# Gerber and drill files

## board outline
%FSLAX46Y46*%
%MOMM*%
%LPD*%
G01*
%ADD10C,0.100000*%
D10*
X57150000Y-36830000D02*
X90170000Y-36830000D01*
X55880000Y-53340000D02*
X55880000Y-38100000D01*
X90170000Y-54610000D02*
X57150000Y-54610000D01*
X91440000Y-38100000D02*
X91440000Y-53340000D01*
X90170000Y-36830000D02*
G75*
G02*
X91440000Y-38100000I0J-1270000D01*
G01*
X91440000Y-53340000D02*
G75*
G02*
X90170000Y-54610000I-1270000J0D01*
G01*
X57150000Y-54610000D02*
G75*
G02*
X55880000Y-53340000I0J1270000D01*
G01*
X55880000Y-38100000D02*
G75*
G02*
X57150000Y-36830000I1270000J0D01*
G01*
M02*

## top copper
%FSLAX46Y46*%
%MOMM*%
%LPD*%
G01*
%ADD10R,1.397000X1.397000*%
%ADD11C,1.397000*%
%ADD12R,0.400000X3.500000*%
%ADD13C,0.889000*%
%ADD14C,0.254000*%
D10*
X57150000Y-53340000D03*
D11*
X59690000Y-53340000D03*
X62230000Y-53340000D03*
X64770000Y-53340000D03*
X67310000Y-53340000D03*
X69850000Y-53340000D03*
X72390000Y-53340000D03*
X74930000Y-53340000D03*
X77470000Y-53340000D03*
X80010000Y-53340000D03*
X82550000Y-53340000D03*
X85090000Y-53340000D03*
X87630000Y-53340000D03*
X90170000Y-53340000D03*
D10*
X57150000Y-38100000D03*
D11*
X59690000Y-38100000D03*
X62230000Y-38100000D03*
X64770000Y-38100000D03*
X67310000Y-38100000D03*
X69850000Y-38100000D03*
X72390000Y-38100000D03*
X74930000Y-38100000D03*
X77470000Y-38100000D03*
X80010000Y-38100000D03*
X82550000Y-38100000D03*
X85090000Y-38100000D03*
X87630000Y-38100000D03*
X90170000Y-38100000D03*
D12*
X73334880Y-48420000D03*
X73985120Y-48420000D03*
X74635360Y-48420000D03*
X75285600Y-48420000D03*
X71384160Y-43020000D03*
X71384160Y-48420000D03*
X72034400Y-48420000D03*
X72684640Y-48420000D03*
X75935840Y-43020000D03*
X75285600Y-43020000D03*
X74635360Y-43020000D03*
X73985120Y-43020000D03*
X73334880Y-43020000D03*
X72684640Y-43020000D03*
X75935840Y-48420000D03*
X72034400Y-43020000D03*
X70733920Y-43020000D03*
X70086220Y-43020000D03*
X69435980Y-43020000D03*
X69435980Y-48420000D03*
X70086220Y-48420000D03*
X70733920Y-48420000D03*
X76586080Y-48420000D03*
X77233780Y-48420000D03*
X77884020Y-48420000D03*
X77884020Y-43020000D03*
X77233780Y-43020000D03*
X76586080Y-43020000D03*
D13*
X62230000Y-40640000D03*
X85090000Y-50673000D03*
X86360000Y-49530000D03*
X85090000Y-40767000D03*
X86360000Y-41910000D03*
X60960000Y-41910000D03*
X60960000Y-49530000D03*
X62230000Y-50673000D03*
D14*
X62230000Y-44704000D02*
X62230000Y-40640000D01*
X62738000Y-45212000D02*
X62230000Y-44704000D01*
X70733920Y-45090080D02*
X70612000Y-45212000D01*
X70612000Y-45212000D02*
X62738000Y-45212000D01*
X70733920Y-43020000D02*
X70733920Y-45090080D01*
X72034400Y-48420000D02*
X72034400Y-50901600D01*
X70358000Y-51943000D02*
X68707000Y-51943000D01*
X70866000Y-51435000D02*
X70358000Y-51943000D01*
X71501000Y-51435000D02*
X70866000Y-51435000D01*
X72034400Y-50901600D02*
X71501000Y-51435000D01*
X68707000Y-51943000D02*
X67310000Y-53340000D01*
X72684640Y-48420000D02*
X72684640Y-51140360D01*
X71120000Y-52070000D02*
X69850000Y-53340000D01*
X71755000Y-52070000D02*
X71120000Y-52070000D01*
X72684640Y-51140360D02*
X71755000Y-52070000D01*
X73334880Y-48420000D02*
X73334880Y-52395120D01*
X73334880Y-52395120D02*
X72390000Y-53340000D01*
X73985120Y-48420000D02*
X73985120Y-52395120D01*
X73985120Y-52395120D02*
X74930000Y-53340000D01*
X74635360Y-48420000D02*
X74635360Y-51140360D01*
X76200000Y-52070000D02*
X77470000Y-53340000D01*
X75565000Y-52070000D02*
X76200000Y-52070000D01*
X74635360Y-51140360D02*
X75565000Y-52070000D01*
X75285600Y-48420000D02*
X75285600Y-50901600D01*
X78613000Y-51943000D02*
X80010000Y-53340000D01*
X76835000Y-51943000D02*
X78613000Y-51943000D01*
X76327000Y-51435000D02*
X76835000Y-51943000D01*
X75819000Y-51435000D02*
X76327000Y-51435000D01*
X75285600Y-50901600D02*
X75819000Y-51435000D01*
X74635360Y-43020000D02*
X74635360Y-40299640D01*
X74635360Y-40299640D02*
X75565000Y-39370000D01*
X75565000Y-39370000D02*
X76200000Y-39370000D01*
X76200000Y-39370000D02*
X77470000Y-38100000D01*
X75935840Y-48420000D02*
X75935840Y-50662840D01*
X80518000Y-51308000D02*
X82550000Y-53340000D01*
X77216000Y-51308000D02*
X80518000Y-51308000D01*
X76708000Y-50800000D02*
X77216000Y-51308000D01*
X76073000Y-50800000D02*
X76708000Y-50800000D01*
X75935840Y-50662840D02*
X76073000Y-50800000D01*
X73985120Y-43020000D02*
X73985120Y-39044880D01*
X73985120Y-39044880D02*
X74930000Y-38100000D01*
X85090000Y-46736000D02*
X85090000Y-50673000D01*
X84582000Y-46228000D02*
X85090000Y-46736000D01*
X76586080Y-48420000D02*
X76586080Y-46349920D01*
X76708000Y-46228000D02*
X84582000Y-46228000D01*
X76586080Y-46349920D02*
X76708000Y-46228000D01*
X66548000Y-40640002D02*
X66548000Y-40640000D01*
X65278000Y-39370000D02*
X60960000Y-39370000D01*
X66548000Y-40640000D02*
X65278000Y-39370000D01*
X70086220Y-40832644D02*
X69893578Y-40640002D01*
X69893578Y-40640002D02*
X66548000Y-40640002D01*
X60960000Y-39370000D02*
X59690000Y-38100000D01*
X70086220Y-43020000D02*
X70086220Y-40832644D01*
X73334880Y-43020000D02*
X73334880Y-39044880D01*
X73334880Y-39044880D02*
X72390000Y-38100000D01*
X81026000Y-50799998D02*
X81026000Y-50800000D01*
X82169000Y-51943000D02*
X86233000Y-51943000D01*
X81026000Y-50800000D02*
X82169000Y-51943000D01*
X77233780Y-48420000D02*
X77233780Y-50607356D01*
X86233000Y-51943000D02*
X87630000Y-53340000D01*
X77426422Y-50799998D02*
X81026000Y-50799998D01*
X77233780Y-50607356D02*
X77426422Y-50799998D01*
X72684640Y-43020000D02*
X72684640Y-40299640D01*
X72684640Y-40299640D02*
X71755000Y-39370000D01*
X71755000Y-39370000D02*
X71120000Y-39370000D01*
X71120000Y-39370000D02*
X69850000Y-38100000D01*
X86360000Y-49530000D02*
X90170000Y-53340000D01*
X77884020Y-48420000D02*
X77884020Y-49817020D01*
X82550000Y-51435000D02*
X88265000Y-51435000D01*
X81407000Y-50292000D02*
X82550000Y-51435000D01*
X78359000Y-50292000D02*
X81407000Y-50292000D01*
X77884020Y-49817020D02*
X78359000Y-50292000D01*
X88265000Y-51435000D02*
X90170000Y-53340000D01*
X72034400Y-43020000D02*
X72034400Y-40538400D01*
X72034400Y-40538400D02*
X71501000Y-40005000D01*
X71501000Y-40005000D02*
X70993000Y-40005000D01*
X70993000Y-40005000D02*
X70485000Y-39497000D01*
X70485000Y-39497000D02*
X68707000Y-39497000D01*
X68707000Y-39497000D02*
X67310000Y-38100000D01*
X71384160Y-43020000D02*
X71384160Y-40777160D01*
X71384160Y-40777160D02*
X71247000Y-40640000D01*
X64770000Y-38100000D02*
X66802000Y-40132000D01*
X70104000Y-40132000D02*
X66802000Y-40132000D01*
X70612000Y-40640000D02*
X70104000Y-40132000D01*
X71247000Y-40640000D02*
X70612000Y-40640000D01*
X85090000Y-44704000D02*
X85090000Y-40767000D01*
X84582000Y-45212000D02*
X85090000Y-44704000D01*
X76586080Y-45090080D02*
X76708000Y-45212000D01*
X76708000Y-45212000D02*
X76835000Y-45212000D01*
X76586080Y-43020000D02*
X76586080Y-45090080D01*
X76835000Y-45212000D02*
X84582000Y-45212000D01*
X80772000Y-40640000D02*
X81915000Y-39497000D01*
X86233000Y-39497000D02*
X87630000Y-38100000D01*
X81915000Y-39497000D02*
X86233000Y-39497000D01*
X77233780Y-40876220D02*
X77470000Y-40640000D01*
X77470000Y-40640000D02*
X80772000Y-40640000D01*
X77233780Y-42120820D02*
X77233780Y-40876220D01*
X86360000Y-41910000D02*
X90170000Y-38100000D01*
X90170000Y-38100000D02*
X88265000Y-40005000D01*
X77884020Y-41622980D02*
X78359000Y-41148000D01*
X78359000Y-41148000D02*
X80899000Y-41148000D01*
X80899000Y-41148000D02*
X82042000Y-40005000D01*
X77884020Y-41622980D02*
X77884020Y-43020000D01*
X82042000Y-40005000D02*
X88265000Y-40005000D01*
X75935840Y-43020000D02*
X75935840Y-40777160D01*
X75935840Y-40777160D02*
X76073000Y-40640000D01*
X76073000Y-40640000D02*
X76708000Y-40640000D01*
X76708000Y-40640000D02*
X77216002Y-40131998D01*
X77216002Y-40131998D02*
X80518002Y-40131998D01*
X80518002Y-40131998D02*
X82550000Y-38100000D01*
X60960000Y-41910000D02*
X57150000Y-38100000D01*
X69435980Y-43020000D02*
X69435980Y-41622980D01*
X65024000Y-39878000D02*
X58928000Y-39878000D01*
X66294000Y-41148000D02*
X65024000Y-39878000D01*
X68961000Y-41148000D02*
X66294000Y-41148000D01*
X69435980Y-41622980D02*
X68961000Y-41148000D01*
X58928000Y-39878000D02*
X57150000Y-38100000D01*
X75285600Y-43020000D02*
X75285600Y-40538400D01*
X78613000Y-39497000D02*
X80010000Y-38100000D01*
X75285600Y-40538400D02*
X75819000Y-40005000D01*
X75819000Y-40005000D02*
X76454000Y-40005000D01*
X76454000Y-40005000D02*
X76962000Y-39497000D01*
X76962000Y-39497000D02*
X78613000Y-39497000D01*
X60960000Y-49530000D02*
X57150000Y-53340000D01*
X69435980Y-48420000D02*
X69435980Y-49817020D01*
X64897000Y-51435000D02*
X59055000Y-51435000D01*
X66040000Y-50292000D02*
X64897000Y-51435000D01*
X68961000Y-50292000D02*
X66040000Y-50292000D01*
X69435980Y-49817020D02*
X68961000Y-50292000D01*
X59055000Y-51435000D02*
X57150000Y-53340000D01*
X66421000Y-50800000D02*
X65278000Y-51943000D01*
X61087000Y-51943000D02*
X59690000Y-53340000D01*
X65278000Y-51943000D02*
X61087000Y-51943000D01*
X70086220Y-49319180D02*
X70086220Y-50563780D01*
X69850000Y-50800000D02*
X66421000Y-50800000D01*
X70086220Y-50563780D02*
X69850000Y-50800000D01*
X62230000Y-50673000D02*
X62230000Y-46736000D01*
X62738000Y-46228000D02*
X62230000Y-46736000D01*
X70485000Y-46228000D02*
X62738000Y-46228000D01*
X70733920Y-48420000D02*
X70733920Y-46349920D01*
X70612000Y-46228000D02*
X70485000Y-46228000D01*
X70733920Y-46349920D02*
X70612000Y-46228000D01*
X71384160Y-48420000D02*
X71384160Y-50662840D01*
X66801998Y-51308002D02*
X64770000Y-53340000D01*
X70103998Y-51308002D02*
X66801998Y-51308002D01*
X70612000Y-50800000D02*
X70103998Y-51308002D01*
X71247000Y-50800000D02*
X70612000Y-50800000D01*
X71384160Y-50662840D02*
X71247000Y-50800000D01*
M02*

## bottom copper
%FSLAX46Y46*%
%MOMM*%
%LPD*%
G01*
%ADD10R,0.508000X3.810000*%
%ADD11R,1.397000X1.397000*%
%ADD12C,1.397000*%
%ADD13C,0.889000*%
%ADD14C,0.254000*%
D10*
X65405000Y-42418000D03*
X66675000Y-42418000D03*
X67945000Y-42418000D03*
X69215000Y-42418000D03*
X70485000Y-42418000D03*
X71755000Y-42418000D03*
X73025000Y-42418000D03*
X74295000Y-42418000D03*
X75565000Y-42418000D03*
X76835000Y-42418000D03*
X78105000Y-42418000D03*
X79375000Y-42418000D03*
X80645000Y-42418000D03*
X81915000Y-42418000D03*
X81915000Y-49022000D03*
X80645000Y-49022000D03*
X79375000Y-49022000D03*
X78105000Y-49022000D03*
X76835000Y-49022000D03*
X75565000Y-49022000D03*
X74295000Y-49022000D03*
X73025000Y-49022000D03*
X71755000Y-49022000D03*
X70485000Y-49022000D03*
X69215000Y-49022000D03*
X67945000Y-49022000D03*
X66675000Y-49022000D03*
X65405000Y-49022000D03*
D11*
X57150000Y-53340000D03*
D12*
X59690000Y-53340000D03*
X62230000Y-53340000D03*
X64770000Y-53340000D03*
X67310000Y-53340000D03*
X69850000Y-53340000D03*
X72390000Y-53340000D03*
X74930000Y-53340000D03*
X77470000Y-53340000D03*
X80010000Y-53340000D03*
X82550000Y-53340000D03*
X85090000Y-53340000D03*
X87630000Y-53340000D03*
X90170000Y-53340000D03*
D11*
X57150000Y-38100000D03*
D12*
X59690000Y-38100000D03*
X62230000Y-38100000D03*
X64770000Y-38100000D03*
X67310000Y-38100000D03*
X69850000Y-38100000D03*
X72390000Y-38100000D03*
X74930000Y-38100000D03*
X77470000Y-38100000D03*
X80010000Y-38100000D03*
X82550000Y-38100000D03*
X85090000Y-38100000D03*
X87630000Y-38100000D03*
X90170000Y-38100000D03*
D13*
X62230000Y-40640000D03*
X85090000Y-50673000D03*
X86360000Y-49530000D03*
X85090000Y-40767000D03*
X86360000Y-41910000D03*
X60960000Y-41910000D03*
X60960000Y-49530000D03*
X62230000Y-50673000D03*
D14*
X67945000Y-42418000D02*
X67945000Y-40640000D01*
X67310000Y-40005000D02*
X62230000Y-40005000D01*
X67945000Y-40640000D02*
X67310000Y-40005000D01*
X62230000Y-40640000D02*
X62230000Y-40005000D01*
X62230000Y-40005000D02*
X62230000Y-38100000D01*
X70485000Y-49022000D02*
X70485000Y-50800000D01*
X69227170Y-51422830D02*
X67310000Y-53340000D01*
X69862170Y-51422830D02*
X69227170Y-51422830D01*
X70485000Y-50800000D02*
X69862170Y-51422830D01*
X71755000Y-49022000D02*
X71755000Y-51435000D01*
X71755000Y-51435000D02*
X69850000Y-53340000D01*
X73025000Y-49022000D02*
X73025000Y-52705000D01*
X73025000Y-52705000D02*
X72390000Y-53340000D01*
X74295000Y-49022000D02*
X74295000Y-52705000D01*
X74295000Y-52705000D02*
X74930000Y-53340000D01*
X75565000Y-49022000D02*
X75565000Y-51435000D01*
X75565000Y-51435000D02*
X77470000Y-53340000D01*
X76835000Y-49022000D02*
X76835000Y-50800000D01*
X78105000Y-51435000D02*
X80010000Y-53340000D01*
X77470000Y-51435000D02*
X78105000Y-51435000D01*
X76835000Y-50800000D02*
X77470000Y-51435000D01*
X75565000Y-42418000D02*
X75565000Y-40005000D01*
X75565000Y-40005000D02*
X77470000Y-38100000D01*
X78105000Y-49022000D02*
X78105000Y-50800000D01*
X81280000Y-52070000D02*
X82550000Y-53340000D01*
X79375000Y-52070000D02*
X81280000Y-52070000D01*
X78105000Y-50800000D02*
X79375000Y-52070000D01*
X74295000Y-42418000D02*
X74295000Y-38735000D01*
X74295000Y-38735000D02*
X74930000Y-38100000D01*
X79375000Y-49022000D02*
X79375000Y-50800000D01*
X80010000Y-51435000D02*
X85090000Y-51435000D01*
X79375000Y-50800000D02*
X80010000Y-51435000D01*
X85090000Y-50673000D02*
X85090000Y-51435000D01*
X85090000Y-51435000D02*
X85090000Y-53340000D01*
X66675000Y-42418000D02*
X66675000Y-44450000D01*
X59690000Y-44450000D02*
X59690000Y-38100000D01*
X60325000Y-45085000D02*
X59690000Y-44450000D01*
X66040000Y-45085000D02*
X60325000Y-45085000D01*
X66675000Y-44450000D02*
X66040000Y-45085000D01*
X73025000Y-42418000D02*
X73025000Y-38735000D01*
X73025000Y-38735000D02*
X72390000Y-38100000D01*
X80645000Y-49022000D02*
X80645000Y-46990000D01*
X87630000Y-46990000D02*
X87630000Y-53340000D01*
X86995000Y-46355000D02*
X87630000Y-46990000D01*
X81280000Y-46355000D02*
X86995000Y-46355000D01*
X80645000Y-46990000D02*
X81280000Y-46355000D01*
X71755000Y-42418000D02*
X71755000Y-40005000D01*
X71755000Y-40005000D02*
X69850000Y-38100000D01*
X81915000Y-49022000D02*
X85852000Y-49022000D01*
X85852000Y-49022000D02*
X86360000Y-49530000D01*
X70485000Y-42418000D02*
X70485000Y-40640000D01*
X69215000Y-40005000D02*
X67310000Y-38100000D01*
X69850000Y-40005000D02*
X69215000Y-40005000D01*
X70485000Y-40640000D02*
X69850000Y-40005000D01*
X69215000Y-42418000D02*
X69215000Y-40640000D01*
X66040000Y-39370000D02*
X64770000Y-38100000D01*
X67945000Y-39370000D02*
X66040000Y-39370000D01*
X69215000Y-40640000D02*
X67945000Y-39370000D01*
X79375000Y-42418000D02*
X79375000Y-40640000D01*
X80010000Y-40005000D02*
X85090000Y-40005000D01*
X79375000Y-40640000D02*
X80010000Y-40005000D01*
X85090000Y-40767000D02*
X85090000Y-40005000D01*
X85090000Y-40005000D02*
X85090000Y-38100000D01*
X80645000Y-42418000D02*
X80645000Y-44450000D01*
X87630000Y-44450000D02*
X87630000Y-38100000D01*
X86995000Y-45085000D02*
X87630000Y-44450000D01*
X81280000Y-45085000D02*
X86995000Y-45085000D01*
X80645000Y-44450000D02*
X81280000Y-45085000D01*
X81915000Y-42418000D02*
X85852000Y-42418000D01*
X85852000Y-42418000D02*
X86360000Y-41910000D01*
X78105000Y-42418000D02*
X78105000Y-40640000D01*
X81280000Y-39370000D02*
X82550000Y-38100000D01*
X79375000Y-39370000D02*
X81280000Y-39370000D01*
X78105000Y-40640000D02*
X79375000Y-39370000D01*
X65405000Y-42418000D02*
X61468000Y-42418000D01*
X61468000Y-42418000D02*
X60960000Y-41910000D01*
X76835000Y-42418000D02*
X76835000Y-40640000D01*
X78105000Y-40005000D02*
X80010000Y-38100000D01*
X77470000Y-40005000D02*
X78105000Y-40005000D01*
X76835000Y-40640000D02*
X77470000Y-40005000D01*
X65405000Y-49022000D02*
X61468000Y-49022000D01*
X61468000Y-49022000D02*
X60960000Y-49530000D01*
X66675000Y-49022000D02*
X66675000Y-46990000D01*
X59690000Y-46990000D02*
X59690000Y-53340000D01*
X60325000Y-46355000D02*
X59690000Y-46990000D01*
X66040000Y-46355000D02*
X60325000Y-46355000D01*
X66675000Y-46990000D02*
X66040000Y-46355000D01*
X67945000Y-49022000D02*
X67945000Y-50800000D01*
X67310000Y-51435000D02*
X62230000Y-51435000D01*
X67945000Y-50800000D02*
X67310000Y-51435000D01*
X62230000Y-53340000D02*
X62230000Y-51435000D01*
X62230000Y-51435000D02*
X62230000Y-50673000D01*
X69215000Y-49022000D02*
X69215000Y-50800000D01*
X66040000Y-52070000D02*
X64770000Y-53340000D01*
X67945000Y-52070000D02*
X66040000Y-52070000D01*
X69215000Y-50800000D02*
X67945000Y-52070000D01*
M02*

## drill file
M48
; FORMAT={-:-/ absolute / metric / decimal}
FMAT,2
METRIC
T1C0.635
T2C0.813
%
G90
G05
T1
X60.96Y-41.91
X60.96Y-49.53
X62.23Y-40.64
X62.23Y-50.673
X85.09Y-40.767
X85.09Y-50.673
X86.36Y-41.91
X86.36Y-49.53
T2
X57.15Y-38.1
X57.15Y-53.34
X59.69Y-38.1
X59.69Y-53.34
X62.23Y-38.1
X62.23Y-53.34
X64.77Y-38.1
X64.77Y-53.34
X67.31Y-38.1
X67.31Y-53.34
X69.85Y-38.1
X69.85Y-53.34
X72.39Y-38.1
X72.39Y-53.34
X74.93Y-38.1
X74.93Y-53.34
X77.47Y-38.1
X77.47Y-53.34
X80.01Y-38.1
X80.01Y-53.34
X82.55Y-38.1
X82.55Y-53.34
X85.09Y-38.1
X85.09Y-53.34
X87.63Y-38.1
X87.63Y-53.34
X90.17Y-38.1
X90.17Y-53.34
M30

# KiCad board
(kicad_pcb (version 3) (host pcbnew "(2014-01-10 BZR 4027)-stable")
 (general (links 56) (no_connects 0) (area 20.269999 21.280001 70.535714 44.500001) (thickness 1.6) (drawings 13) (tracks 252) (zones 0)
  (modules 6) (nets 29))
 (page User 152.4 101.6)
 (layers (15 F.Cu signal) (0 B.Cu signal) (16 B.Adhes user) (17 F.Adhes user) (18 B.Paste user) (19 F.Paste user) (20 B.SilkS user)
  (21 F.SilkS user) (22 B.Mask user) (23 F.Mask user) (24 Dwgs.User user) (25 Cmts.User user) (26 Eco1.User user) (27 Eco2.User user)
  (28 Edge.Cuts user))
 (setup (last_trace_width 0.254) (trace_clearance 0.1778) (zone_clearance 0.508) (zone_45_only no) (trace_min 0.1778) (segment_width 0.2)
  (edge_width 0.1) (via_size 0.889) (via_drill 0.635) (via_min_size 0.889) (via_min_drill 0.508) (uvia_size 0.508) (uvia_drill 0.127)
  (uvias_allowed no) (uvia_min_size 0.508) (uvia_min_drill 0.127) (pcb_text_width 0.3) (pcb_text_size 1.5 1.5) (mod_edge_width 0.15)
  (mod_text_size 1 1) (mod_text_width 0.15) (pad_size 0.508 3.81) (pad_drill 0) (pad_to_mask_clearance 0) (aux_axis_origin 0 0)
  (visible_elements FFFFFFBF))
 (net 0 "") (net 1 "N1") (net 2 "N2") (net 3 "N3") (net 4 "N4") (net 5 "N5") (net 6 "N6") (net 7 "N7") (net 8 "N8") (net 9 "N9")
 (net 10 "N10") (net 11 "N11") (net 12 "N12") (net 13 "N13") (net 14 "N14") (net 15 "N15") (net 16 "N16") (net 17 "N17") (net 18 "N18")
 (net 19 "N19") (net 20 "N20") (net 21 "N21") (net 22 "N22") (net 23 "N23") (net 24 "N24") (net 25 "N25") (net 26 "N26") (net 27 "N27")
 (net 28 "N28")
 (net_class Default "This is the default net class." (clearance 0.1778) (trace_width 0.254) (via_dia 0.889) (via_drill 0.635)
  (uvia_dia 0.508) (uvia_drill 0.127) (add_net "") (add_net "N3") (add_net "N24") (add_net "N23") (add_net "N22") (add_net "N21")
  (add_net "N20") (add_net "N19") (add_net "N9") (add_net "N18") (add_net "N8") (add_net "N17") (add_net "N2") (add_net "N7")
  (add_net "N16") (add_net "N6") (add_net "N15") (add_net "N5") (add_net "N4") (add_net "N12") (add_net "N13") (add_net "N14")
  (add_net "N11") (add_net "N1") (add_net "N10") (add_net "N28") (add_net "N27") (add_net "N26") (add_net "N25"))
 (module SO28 (layer B.Cu) (at 73.66 45.72)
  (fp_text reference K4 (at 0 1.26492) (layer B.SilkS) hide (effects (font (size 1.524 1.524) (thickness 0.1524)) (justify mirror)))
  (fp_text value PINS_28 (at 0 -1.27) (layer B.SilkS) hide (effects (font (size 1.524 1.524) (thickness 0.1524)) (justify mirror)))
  (pad 1 smd rect (at -8.255 -3.302) (size 0.508 3.81) (layers B.Cu B.Paste B.Mask) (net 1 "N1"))
  (pad 2 smd rect (at -6.985 -3.302) (size 0.508 3.81) (layers B.Cu B.Paste B.Mask) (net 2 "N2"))
  (pad 3 smd rect (at -5.715 -3.302) (size 0.508 3.81) (layers B.Cu B.Paste B.Mask) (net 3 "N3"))
  (pad 4 smd rect (at -4.445 -3.302) (size 0.508 3.81) (layers B.Cu B.Paste B.Mask) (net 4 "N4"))
  (pad 5 smd rect (at -3.175 -3.302) (size 0.508 3.81) (layers B.Cu B.Paste B.Mask) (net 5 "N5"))
  (pad 6 smd rect (at -1.905 -3.302) (size 0.508 3.81) (layers B.Cu B.Paste B.Mask) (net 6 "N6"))
  (pad 7 smd rect (at -0.635 -3.302) (size 0.508 3.81) (layers B.Cu B.Paste B.Mask) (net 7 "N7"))
  (pad 8 smd rect (at 0.635 -3.302) (size 0.508 3.81) (layers B.Cu B.Paste B.Mask) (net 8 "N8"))
  (pad 9 smd rect (at 1.905 -3.302) (size 0.508 3.81) (layers B.Cu B.Paste B.Mask) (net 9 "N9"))
  (pad 10 smd rect (at 3.175 -3.302) (size 0.508 3.81) (layers B.Cu B.Paste B.Mask) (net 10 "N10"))
  (pad 11 smd rect (at 4.445 -3.302) (size 0.508 3.81) (layers B.Cu B.Paste B.Mask) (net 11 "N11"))
  (pad 12 smd rect (at 5.715 -3.302) (size 0.508 3.81) (layers B.Cu B.Paste B.Mask) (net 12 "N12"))
  (pad 13 smd rect (at 6.985 -3.302) (size 0.508 3.81) (layers B.Cu B.Paste B.Mask) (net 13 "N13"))
  (pad 14 smd rect (at 8.255 -3.302) (size 0.508 3.81) (layers B.Cu B.Paste B.Mask) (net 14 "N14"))
  (pad 15 smd rect (at 8.255 3.302) (size 0.508 3.81) (layers B.Cu B.Paste B.Mask) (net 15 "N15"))
  (pad 16 smd rect (at 6.985 3.302) (size 0.508 3.81) (layers B.Cu B.Paste B.Mask) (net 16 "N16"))
  (pad 17 smd rect (at 5.715 3.302) (size 0.508 3.81) (layers B.Cu B.Paste B.Mask) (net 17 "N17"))
  (pad 18 smd rect (at 4.445 3.302) (size 0.508 3.81) (layers B.Cu B.Paste B.Mask) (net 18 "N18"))
  (pad 19 smd rect (at 3.175 3.302) (size 0.508 3.81) (layers B.Cu B.Paste B.Mask) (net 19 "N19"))
  (pad 20 smd rect (at 1.905 3.302) (size 0.508 3.81) (layers B.Cu B.Paste B.Mask) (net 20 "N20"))
  (pad 21 smd rect (at 0.635 3.302) (size 0.508 3.81) (layers B.Cu B.Paste B.Mask) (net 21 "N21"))
  (pad 22 smd rect (at -0.635 3.302) (size 0.508 3.81) (layers B.Cu B.Paste B.Mask) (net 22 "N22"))
  (pad 23 smd rect (at -1.905 3.302) (size 0.508 3.81) (layers B.Cu B.Paste B.Mask) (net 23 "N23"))
  (pad 24 smd rect (at -3.175 3.302) (size 0.508 3.81) (layers B.Cu B.Paste B.Mask) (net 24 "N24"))
  (pad 25 smd rect (at -4.445 3.302) (size 0.508 3.81) (layers B.Cu B.Paste B.Mask) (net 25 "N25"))
  (pad 26 smd rect (at -5.715 3.302) (size 0.508 3.81) (layers B.Cu B.Paste B.Mask) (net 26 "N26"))
  (pad 27 smd rect (at -6.985 3.302) (size 0.508 3.81) (layers B.Cu B.Paste B.Mask) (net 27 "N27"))
  (pad 28 smd rect (at -8.255 3.302) (size 0.508 3.81) (layers B.Cu B.Paste B.Mask) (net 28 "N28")))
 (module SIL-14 (layer F.Cu) (at 73.66 53.34)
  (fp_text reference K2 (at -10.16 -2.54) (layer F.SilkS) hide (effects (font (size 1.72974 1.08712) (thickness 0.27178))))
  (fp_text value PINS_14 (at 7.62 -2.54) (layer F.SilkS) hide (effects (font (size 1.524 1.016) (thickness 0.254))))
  (pad 1 thru_hole rect (at -16.51 0) (size 1.397 1.397) (drill 0.8128) (layers *.Cu *.Mask F.SilkS) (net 28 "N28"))
  (pad 2 thru_hole circle (at -13.97 0) (size 1.397 1.397) (drill 0.8128) (layers *.Cu *.Mask F.SilkS) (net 27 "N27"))
  (pad 3 thru_hole circle (at -11.43 0) (size 1.397 1.397) (drill 0.8128) (layers *.Cu *.Mask F.SilkS) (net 26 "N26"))
  (pad 4 thru_hole circle (at -8.89 0) (size 1.397 1.397) (drill 0.8128) (layers *.Cu *.Mask F.SilkS) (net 25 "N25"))
  (pad 5 thru_hole circle (at -6.35 0) (size 1.397 1.397) (drill 0.8128) (layers *.Cu *.Mask F.SilkS) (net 24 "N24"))
  (pad 6 thru_hole circle (at -3.81 0) (size 1.397 1.397) (drill 0.8128) (layers *.Cu *.Mask F.SilkS) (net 23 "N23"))
  (pad 7 thru_hole circle (at -1.27 0) (size 1.397 1.397) (drill 0.8128) (layers *.Cu *.Mask F.SilkS) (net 22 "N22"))
  (pad 8 thru_hole circle (at 1.27 0) (size 1.397 1.397) (drill 0.8128) (layers *.Cu *.Mask F.SilkS) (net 21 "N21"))
  (pad 9 thru_hole circle (at 3.81 0) (size 1.397 1.397) (drill 0.8128) (layers *.Cu *.Mask F.SilkS) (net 20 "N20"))
  (pad 10 thru_hole circle (at 6.35 0) (size 1.397 1.397) (drill 0.8128) (layers *.Cu *.Mask F.SilkS) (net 19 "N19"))
  (pad 11 thru_hole circle (at 8.89 0) (size 1.397 1.397) (drill 0.8128) (layers *.Cu *.Mask F.SilkS) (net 18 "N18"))
  (pad 12 thru_hole circle (at 11.43 0) (size 1.397 1.397) (drill 0.8128) (layers *.Cu *.Mask F.SilkS) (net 17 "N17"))
  (pad 13 thru_hole circle (at 13.97 0) (size 1.397 1.397) (drill 0.8128) (layers *.Cu *.Mask F.SilkS) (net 16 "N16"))
  (pad 14 thru_hole circle (at 16.51 0) (size 1.397 1.397) (drill 0.8128) (layers *.Cu *.Mask F.SilkS) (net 15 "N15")))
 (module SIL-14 (layer F.Cu) (at 73.66 38.1)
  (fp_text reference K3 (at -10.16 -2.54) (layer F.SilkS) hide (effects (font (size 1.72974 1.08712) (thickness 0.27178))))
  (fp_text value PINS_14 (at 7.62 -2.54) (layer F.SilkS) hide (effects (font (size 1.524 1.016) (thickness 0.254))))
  (pad 1 thru_hole rect (at -16.51 0) (size 1.397 1.397) (drill 0.8128) (layers *.Cu *.Mask F.SilkS) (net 1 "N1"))
  (pad 2 thru_hole circle (at -13.97 0) (size 1.397 1.397) (drill 0.8128) (layers *.Cu *.Mask F.SilkS) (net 2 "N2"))
  (pad 3 thru_hole circle (at -11.43 0) (size 1.397 1.397) (drill 0.8128) (layers *.Cu *.Mask F.SilkS) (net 3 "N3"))
  (pad 4 thru_hole circle (at -8.89 0) (size 1.397 1.397) (drill 0.8128) (layers *.Cu *.Mask F.SilkS) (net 4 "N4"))
  (pad 5 thru_hole circle (at -6.35 0) (size 1.397 1.397) (drill 0.8128) (layers *.Cu *.Mask F.SilkS) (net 5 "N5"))
  (pad 6 thru_hole circle (at -3.81 0) (size 1.397 1.397) (drill 0.8128) (layers *.Cu *.Mask F.SilkS) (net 6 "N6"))
  (pad 7 thru_hole circle (at -1.27 0) (size 1.397 1.397) (drill 0.8128) (layers *.Cu *.Mask F.SilkS) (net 7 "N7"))
  (pad 8 thru_hole circle (at 1.27 0) (size 1.397 1.397) (drill 0.8128) (layers *.Cu *.Mask F.SilkS) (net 8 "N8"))
  (pad 9 thru_hole circle (at 3.81 0) (size 1.397 1.397) (drill 0.8128) (layers *.Cu *.Mask F.SilkS) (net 9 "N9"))
  (pad 10 thru_hole circle (at 6.35 0) (size 1.397 1.397) (drill 0.8128) (layers *.Cu *.Mask F.SilkS) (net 10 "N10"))
  (pad 11 thru_hole circle (at 8.89 0) (size 1.397 1.397) (drill 0.8128) (layers *.Cu *.Mask F.SilkS) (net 11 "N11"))
  (pad 12 thru_hole circle (at 11.43 0) (size 1.397 1.397) (drill 0.8128) (layers *.Cu *.Mask F.SilkS) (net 12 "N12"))
  (pad 13 thru_hole circle (at 13.97 0) (size 1.397 1.397) (drill 0.8128) (layers *.Cu *.Mask F.SilkS) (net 13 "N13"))
  (pad 14 thru_hole circle (at 16.51 0) (size 1.397 1.397) (drill 0.8128) (layers *.Cu *.Mask F.SilkS) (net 14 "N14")))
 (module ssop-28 (layer F.Cu) (at 73.66 45.72)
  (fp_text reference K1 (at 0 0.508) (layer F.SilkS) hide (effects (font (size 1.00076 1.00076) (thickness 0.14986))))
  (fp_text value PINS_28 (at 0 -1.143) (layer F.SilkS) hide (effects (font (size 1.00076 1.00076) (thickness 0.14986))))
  (pad 7 smd rect (at -0.32512 2.7) (size 0.4 3.5) (layers F.Cu F.Paste F.Mask) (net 22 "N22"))
  (pad 8 smd rect (at 0.32512 2.7) (size 0.4 3.5) (layers F.Cu F.Paste F.Mask) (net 21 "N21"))
  (pad 9 smd rect (at 0.97536 2.7) (size 0.4 3.5) (layers F.Cu F.Paste F.Mask) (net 20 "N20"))
  (pad 10 smd rect (at 1.6256 2.7) (size 0.4 3.5) (layers F.Cu F.Paste F.Mask) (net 19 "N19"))
  (pad 25 smd rect (at -2.27584 -2.7) (size 0.4 3.5) (layers F.Cu F.Paste F.Mask) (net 4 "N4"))
  (pad 4 smd rect (at -2.27584 2.7) (size 0.4 3.5) (layers F.Cu F.Paste F.Mask) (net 25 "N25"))
  (pad 5 smd rect (at -1.6256 2.7) (size 0.4 3.5) (layers F.Cu F.Paste F.Mask) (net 24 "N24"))
  (pad 6 smd rect (at -0.97536 2.7) (size 0.4 3.5) (layers F.Cu F.Paste F.Mask) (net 23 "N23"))
  (pad 18 smd rect (at 2.27584 -2.7) (size 0.4 3.5) (layers F.Cu F.Paste F.Mask) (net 11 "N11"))
  (pad 19 smd rect (at 1.6256 -2.7) (size 0.4 3.5) (layers F.Cu F.Paste F.Mask) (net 10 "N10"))
  (pad 20 smd rect (at 0.97536 -2.7) (size 0.4 3.5) (layers F.Cu F.Paste F.Mask) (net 9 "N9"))
  (pad 21 smd rect (at 0.32512 -2.7) (size 0.4 3.5) (layers F.Cu F.Paste F.Mask) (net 8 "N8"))
  (pad 22 smd rect (at -0.32512 -2.7) (size 0.4 3.5) (layers F.Cu F.Paste F.Mask) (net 7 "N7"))
  (pad 23 smd rect (at -0.97536 -2.7) (size 0.4 3.5) (layers F.Cu F.Paste F.Mask) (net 6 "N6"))
  (pad 11 smd rect (at 2.27584 2.7) (size 0.4 3.5) (layers F.Cu F.Paste F.Mask) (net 18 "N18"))
  (pad 24 smd rect (at -1.6256 -2.7) (size 0.4 3.5) (layers F.Cu F.Paste F.Mask) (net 5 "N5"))
  (pad 26 smd rect (at -2.92608 -2.7) (size 0.4 3.5) (layers F.Cu F.Paste F.Mask) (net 3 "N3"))
  (pad 27 smd rect (at -3.57378 -2.7) (size 0.4 3.5) (layers F.Cu F.Paste F.Mask) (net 2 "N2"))
  (pad 28 smd rect (at -4.22402 -2.7) (size 0.4 3.5) (layers F.Cu F.Paste F.Mask) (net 1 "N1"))
  (pad 1 smd rect (at -4.22402 2.7) (size 0.4 3.5) (layers F.Cu F.Paste F.Mask) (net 28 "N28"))
  (pad 2 smd rect (at -3.57378 2.7) (size 0.4 3.5) (layers F.Cu F.Paste F.Mask) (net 27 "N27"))
  (pad 3 smd rect (at -2.92608 2.7) (size 0.4 3.5) (layers F.Cu F.Paste F.Mask) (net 26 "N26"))
  (pad 12 smd rect (at 2.92608 2.7) (size 0.4 3.5) (layers F.Cu F.Paste F.Mask) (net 17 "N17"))
  (pad 13 smd rect (at 3.57378 2.7) (size 0.4 3.5) (layers F.Cu F.Paste F.Mask) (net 16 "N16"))
  (pad 14 smd rect (at 4.22402 2.7) (size 0.4 3.5) (layers F.Cu F.Paste F.Mask) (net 15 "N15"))
  (pad 15 smd rect (at 4.22402 -2.7) (size 0.4 3.5) (layers F.Cu F.Paste F.Mask) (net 14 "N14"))
  (pad 16 smd rect (at 3.57378 -2.7) (size 0.4 3.5) (layers F.Cu F.Paste F.Mask) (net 13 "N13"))
  (pad 17 smd rect (at 2.92608 -2.7) (size 0.4 3.5) (layers F.Cu F.Paste F.Mask) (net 12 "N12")))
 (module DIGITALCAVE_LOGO (layer F.Cu) (at 59.055 45.72)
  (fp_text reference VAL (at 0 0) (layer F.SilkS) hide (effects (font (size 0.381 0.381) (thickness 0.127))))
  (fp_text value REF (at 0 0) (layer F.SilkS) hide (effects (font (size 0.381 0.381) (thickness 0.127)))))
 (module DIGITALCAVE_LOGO (layer B.Cu) (at 59.055 45.72)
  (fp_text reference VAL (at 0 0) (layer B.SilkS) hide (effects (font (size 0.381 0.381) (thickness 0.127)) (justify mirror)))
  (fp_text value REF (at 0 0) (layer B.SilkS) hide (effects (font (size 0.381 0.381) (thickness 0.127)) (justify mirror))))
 (gr_line (start 57.15 36.83) (end 90.17 36.83) (angle 90) (layer Edge.Cuts) (width 0.1))
 (gr_line (start 55.88 53.34) (end 55.88 38.1) (angle 90) (layer Edge.Cuts) (width 0.1))
 (gr_line (start 90.17 54.61) (end 57.15 54.61) (angle 90) (layer Edge.Cuts) (width 0.1))
 (gr_line (start 91.44 38.1) (end 91.44 53.34) (angle 90) (layer Edge.Cuts) (width 0.1))
 (gr_arc (start 90.17 38.1) (end 90.17 36.83) (angle 90) (layer Edge.Cuts) (width 0.1))
 (gr_arc (start 90.17 53.34) (end 91.44 53.34) (angle 90) (layer Edge.Cuts) (width 0.1))
 (gr_arc (start 57.15 53.34) (end 57.15 54.61) (angle 90) (layer Edge.Cuts) (width 0.1))
 (gr_arc (start 57.15 38.1) (end 55.88 38.1) (angle 90) (layer Edge.Cuts) (width 0.1))
 (segment (start 67.945 42.418) (end 67.945 40.64) (width 0.254) (layer B.Cu) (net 3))
 (segment (start 67.31 40.005) (end 62.23 40.005) (width 0.254) (layer B.Cu) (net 3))
 (segment (start 67.945 40.64) (end 67.31 40.005) (width 0.254) (layer B.Cu) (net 3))
 (segment (start 62.23 44.704) (end 62.23 40.64) (width 0.254) (layer F.Cu) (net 3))
 (via (at 62.23 40.64) (size 0.889) (layers F.Cu B.Cu) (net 3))
 (segment (start 62.738 45.212) (end 62.23 44.704) (width 0.254) (layer F.Cu) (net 3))
 (segment (start 70.73392 45.09008) (end 70.612 45.212) (width 0.254) (layer F.Cu) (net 3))
 (segment (start 70.612 45.212) (end 62.738 45.212) (width 0.254) (layer F.Cu) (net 3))
 (segment (start 62.23 40.64) (end 62.23 40.005) (width 0.254) (layer B.Cu) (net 3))
 (segment (start 62.23 40.005) (end 62.23 38.1) (width 0.254) (layer B.Cu) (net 3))
 (segment (start 70.73392 43.02) (end 70.73392 45.09008) (width 0.254) (layer F.Cu) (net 3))
 (segment (start 70.485 49.022) (end 70.485 50.8) (width 0.254) (layer B.Cu) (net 24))
 (segment (start 69.22717 51.42283) (end 67.31 53.34) (width 0.254) (layer B.Cu) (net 24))
 (segment (start 69.86217 51.42283) (end 69.22717 51.42283) (width 0.254) (layer B.Cu) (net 24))
 (segment (start 70.485 50.8) (end 69.86217 51.42283) (width 0.254) (layer B.Cu) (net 24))
 (segment (start 72.0344 48.42) (end 72.0344 50.9016) (width 0.254) (layer F.Cu) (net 24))
 (segment (start 70.358 51.943) (end 68.707 51.943) (width 0.254) (layer F.Cu) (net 24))
 (segment (start 70.866 51.435) (end 70.358 51.943) (width 0.254) (layer F.Cu) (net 24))
 (segment (start 71.501 51.435) (end 70.866 51.435) (width 0.254) (layer F.Cu) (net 24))
 (segment (start 72.0344 50.9016) (end 71.501 51.435) (width 0.254) (layer F.Cu) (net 24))
 (segment (start 68.707 51.943) (end 67.31 53.34) (width 0.254) (layer F.Cu) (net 24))
 (segment (start 71.755 49.022) (end 71.755 51.435) (width 0.254) (layer B.Cu) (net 23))
 (segment (start 71.755 51.435) (end 69.85 53.34) (width 0.254) (layer B.Cu) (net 23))
 (segment (start 72.68464 48.42) (end 72.68464 51.14036) (width 0.254) (layer F.Cu) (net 23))
 (segment (start 71.12 52.07) (end 69.85 53.34) (width 0.254) (layer F.Cu) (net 23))
 (segment (start 71.755 52.07) (end 71.12 52.07) (width 0.254) (layer F.Cu) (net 23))
 (segment (start 72.68464 51.14036) (end 71.755 52.07) (width 0.254) (layer F.Cu) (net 23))
 (segment (start 73.025 49.022) (end 73.025 52.705) (width 0.254) (layer B.Cu) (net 22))
 (segment (start 73.025 52.705) (end 72.39 53.34) (width 0.254) (layer B.Cu) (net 22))
 (segment (start 73.33488 48.42) (end 73.33488 52.39512) (width 0.254) (layer F.Cu) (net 22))
 (segment (start 73.33488 52.39512) (end 72.39 53.34) (width 0.254) (layer F.Cu) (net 22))
 (segment (start 74.295 49.022) (end 74.295 52.705) (width 0.254) (layer B.Cu) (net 21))
 (segment (start 74.295 52.705) (end 74.93 53.34) (width 0.254) (layer B.Cu) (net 21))
 (segment (start 73.98512 48.42) (end 73.98512 52.39512) (width 0.254) (layer F.Cu) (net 21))
 (segment (start 73.98512 52.39512) (end 74.93 53.34) (width 0.254) (layer F.Cu) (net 21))
 (segment (start 75.565 49.022) (end 75.565 51.435) (width 0.254) (layer B.Cu) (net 20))
 (segment (start 75.565 51.435) (end 77.47 53.34) (width 0.254) (layer B.Cu) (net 20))
 (segment (start 74.63536 48.42) (end 74.63536 51.14036) (width 0.254) (layer F.Cu) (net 20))
 (segment (start 76.2 52.07) (end 77.47 53.34) (width 0.254) (layer F.Cu) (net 20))
 (segment (start 75.565 52.07) (end 76.2 52.07) (width 0.254) (layer F.Cu) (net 20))
 (segment (start 74.63536 51.14036) (end 75.565 52.07) (width 0.254) (layer F.Cu) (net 20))
 (segment (start 76.835 49.022) (end 76.835 50.8) (width 0.254) (layer B.Cu) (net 19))
 (segment (start 78.105 51.435) (end 80.01 53.34) (width 0.254) (layer B.Cu) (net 19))
 (segment (start 77.47 51.435) (end 78.105 51.435) (width 0.254) (layer B.Cu) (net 19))
 (segment (start 76.835 50.8) (end 77.47 51.435) (width 0.254) (layer B.Cu) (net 19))
 (segment (start 75.2856 48.42) (end 75.2856 50.9016) (width 0.254) (layer F.Cu) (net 19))
 (segment (start 78.613 51.943) (end 80.01 53.34) (width 0.254) (layer F.Cu) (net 19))
 (segment (start 76.835 51.943) (end 78.613 51.943) (width 0.254) (layer F.Cu) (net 19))
 (segment (start 76.327 51.435) (end 76.835 51.943) (width 0.254) (layer F.Cu) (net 19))
 (segment (start 75.819 51.435) (end 76.327 51.435) (width 0.254) (layer F.Cu) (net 19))
 (segment (start 75.2856 50.9016) (end 75.819 51.435) (width 0.254) (layer F.Cu) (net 19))
 (segment (start 75.565 42.418) (end 75.565 40.005) (width 0.254) (layer B.Cu) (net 9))
 (segment (start 75.565 40.005) (end 77.47 38.1) (width 0.254) (layer B.Cu) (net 9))
 (segment (start 74.63536 43.02) (end 74.63536 40.29964) (width 0.254) (layer F.Cu) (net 9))
 (segment (start 74.63536 40.29964) (end 75.565 39.37) (width 0.254) (layer F.Cu) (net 9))
 (segment (start 75.565 39.37) (end 76.2 39.37) (width 0.254) (layer F.Cu) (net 9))
 (segment (start 76.2 39.37) (end 77.47 38.1) (width 0.254) (layer F.Cu) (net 9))
 (segment (start 78.105 49.022) (end 78.105 50.8) (width 0.254) (layer B.Cu) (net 18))
 (segment (start 81.28 52.07) (end 82.55 53.34) (width 0.254) (layer B.Cu) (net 18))
 (segment (start 79.375 52.07) (end 81.28 52.07) (width 0.254) (layer B.Cu) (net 18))
 (segment (start 78.105 50.8) (end 79.375 52.07) (width 0.254) (layer B.Cu) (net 18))
 (segment (start 75.93584 48.42) (end 75.93584 50.66284) (width 0.254) (layer F.Cu) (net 18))
 (segment (start 80.518 51.308) (end 82.55 53.34) (width 0.254) (layer F.Cu) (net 18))
 (segment (start 77.216 51.308) (end 80.518 51.308) (width 0.254) (layer F.Cu) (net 18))
 (segment (start 76.708 50.8) (end 77.216 51.308) (width 0.254) (layer F.Cu) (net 18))
 (segment (start 76.073 50.8) (end 76.708 50.8) (width 0.254) (layer F.Cu) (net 18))
 (segment (start 75.93584 50.66284) (end 76.073 50.8) (width 0.254) (layer F.Cu) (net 18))
 (segment (start 74.295 42.418) (end 74.295 38.735) (width 0.254) (layer B.Cu) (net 8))
 (segment (start 74.295 38.735) (end 74.93 38.1) (width 0.254) (layer B.Cu) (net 8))
 (segment (start 73.98512 43.02) (end 73.98512 39.04488) (width 0.254) (layer F.Cu) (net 8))
 (segment (start 73.98512 39.04488) (end 74.93 38.1) (width 0.254) (layer F.Cu) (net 8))
 (segment (start 79.375 49.022) (end 79.375 50.8) (width 0.254) (layer B.Cu) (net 17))
 (segment (start 80.01 51.435) (end 85.09 51.435) (width 0.254) (layer B.Cu) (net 17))
 (segment (start 79.375 50.8) (end 80.01 51.435) (width 0.254) (layer B.Cu) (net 17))
 (segment (start 85.09 46.736) (end 85.09 50.673) (width 0.254) (layer F.Cu) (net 17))
 (via (at 85.09 50.673) (size 0.889) (layers F.Cu B.Cu) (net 17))
 (segment (start 84.582 46.228) (end 85.09 46.736) (width 0.254) (layer F.Cu) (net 17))
 (segment (start 76.58608 48.42) (end 76.58608 46.34992) (width 0.254) (layer F.Cu) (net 17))
 (segment (start 85.09 50.673) (end 85.09 51.435) (width 0.254) (layer B.Cu) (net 17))
 (segment (start 85.09 51.435) (end 85.09 53.34) (width 0.254) (layer B.Cu) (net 17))
 (segment (start 76.708 46.228) (end 84.582 46.228) (width 0.254) (layer F.Cu) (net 17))
 (segment (start 76.58608 46.34992) (end 76.708 46.228) (width 0.254) (layer F.Cu) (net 17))
 (segment (start 66.675 42.418) (end 66.675 44.45) (width 0.254) (layer B.Cu) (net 2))
 (segment (start 59.69 44.45) (end 59.69 38.1) (width 0.254) (layer B.Cu) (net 2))
 (segment (start 60.325 45.085) (end 59.69 44.45) (width 0.254) (layer B.Cu) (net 2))
 (segment (start 66.04 45.085) (end 60.325 45.085) (width 0.254) (layer B.Cu) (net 2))
 (segment (start 66.675 44.45) (end 66.04 45.085) (width 0.254) (layer B.Cu) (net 2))
 (segment (start 66.548 40.640002) (end 66.548 40.64) (width 0.254) (layer F.Cu) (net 2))
 (segment (start 65.278 39.37) (end 60.96 39.37) (width 0.254) (layer F.Cu) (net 2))
 (segment (start 66.548 40.64) (end 65.278 39.37) (width 0.254) (layer F.Cu) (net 2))
 (segment (start 70.08622 40.832644) (end 69.893578 40.640002) (width 0.254) (layer F.Cu) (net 2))
 (segment (start 69.893578 40.640002) (end 66.548 40.640002) (width 0.254) (layer F.Cu) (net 2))
 (segment (start 60.96 39.37) (end 59.69 38.1) (width 0.254) (layer F.Cu) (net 2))
 (segment (start 70.08622 43.02) (end 70.08622 40.832644) (width 0.254) (layer F.Cu) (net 2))
 (segment (start 73.025 42.418) (end 73.025 38.735) (width 0.254) (layer B.Cu) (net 7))
 (segment (start 73.025 38.735) (end 72.39 38.1) (width 0.254) (layer B.Cu) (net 7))
 (segment (start 73.33488 43.02) (end 73.33488 39.04488) (width 0.254) (layer F.Cu) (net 7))
 (segment (start 73.33488 39.04488) (end 72.39 38.1) (width 0.254) (layer F.Cu) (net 7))
 (segment (start 80.645 49.022) (end 80.645 46.99) (width 0.254) (layer B.Cu) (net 16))
 (segment (start 87.63 46.99) (end 87.63 53.34) (width 0.254) (layer B.Cu) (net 16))
 (segment (start 86.995 46.355) (end 87.63 46.99) (width 0.254) (layer B.Cu) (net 16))
 (segment (start 81.28 46.355) (end 86.995 46.355) (width 0.254) (layer B.Cu) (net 16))
 (segment (start 80.645 46.99) (end 81.28 46.355) (width 0.254) (layer B.Cu) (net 16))
 (segment (start 81.026 50.799998) (end 81.026 50.8) (width 0.254) (layer F.Cu) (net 16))
 (segment (start 82.169 51.943) (end 86.233 51.943) (width 0.254) (layer F.Cu) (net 16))
 (segment (start 81.026 50.8) (end 82.169 51.943) (width 0.254) (layer F.Cu) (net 16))
 (segment (start 77.23378 48.42) (end 77.23378 50.607356) (width 0.254) (layer F.Cu) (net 16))
 (segment (start 86.233 51.943) (end 87.63 53.34) (width 0.254) (layer F.Cu) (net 16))
 (segment (start 77.426422 50.799998) (end 81.026 50.799998) (width 0.254) (layer F.Cu) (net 16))
 (segment (start 77.23378 50.607356) (end 77.426422 50.799998) (width 0.254) (layer F.Cu) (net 16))
 (segment (start 71.755 42.418) (end 71.755 40.005) (width 0.254) (layer B.Cu) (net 6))
 (segment (start 71.755 40.005) (end 69.85 38.1) (width 0.254) (layer B.Cu) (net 6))
 (segment (start 72.68464 43.02) (end 72.68464 40.29964) (width 0.254) (layer F.Cu) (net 6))
 (segment (start 72.68464 40.29964) (end 71.755 39.37) (width 0.254) (layer F.Cu) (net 6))
 (segment (start 71.755 39.37) (end 71.12 39.37) (width 0.254) (layer F.Cu) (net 6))
 (segment (start 71.12 39.37) (end 69.85 38.1) (width 0.254) (layer F.Cu) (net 6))
 (segment (start 81.915 49.022) (end 85.852 49.022) (width 0.254) (layer B.Cu) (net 15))
 (segment (start 86.36 49.53) (end 90.17 53.34) (width 0.254) (layer F.Cu) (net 15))
 (via (at 86.36 49.53) (size 0.889) (layers F.Cu B.Cu) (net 15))
 (segment (start 85.852 49.022) (end 86.36 49.53) (width 0.254) (layer B.Cu) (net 15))
 (segment (start 77.88402 48.42) (end 77.88402 49.81702) (width 0.254) (layer F.Cu) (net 15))
 (segment (start 82.55 51.435) (end 88.265 51.435) (width 0.254) (layer F.Cu) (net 15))
 (segment (start 81.407 50.292) (end 82.55 51.435) (width 0.254) (layer F.Cu) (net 15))
 (segment (start 78.359 50.292) (end 81.407 50.292) (width 0.254) (layer F.Cu) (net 15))
 (segment (start 77.88402 49.81702) (end 78.359 50.292) (width 0.254) (layer F.Cu) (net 15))
 (segment (start 88.265 51.435) (end 90.17 53.34) (width 0.254) (layer F.Cu) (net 15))
 (segment (start 70.485 42.418) (end 70.485 40.64) (width 0.254) (layer B.Cu) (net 5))
 (segment (start 69.215 40.005) (end 67.31 38.1) (width 0.254) (layer B.Cu) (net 5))
 (segment (start 69.85 40.005) (end 69.215 40.005) (width 0.254) (layer B.Cu) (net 5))
 (segment (start 70.485 40.64) (end 69.85 40.005) (width 0.254) (layer B.Cu) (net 5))
 (segment (start 72.0344 43.02) (end 72.0344 40.5384) (width 0.254) (layer F.Cu) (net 5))
 (segment (start 72.0344 40.5384) (end 71.501 40.005) (width 0.254) (layer F.Cu) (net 5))
 (segment (start 71.501 40.005) (end 70.993 40.005) (width 0.254) (layer F.Cu) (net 5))
 (segment (start 70.993 40.005) (end 70.485 39.497) (width 0.254) (layer F.Cu) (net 5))
 (segment (start 70.485 39.497) (end 68.707 39.497) (width 0.254) (layer F.Cu) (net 5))
 (segment (start 68.707 39.497) (end 67.31 38.1) (width 0.254) (layer F.Cu) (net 5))
 (segment (start 69.215 42.418) (end 69.215 40.64) (width 0.254) (layer B.Cu) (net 4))
 (segment (start 66.04 39.37) (end 64.77 38.1) (width 0.254) (layer B.Cu) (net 4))
 (segment (start 67.945 39.37) (end 66.04 39.37) (width 0.254) (layer B.Cu) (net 4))
 (segment (start 69.215 40.64) (end 67.945 39.37) (width 0.254) (layer B.Cu) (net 4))
 (segment (start 71.38416 43.02) (end 71.38416 40.77716) (width 0.254) (layer F.Cu) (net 4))
 (segment (start 71.38416 40.77716) (end 71.247 40.64) (width 0.254) (layer F.Cu) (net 4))
 (segment (start 64.77 38.1) (end 66.802 40.132) (width 0.254) (layer F.Cu) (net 4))
 (segment (start 70.104 40.132) (end 66.802 40.132) (width 0.254) (layer F.Cu) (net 4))
 (segment (start 70.612 40.64) (end 70.104 40.132) (width 0.254) (layer F.Cu) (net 4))
 (segment (start 71.247 40.64) (end 70.612 40.64) (width 0.254) (layer F.Cu) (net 4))
 (segment (start 79.375 42.418) (end 79.375 40.64) (width 0.254) (layer B.Cu) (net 12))
 (segment (start 80.01 40.005) (end 85.09 40.005) (width 0.254) (layer B.Cu) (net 12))
 (segment (start 79.375 40.64) (end 80.01 40.005) (width 0.254) (layer B.Cu) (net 12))
 (segment (start 85.09 44.704) (end 85.09 40.767) (width 0.254) (layer F.Cu) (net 12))
 (via (at 85.09 40.767) (size 0.889) (layers F.Cu B.Cu) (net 12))
 (segment (start 84.582 45.212) (end 85.09 44.704) (width 0.254) (layer F.Cu) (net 12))
 (segment (start 76.58608 45.09008) (end 76.708 45.212) (width 0.254) (layer F.Cu) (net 12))
 (segment (start 76.708 45.212) (end 76.835 45.212) (width 0.254) (layer F.Cu) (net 12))
 (segment (start 76.58608 43.02) (end 76.58608 45.09008) (width 0.254) (layer F.Cu) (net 12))
 (segment (start 76.835 45.212) (end 84.582 45.212) (width 0.254) (layer F.Cu) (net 12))
 (segment (start 85.09 40.767) (end 85.09 40.005) (width 0.254) (layer B.Cu) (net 12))
 (segment (start 85.09 40.005) (end 85.09 38.1) (width 0.254) (layer B.Cu) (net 12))
 (segment (start 80.645 42.418) (end 80.645 44.45) (width 0.254) (layer B.Cu) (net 13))
 (segment (start 87.63 44.45) (end 87.63 38.1) (width 0.254) (layer B.Cu) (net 13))
 (segment (start 86.995 45.085) (end 87.63 44.45) (width 0.254) (layer B.Cu) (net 13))
 (segment (start 81.28 45.085) (end 86.995 45.085) (width 0.254) (layer B.Cu) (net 13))
 (segment (start 80.645 44.45) (end 81.28 45.085) (width 0.254) (layer B.Cu) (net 13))
 (segment (start 80.772 40.64) (end 81.915 39.497) (width 0.254) (layer F.Cu) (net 13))
 (segment (start 86.233 39.497) (end 87.63 38.1) (width 0.254) (layer F.Cu) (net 13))
 (segment (start 81.915 39.497) (end 86.233 39.497) (width 0.254) (layer F.Cu) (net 13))
 (segment (start 77.23378 40.87622) (end 77.47 40.64) (width 0.254) (layer F.Cu) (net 13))
 (segment (start 77.47 40.64) (end 80.772 40.64) (width 0.254) (layer F.Cu) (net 13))
 (segment (start 77.23378 42.12082) (end 77.23378 40.87622) (width 0.254) (layer F.Cu) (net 13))
 (segment (start 81.915 42.418) (end 85.852 42.418) (width 0.254) (layer B.Cu) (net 14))
 (segment (start 86.36 41.91) (end 90.17 38.1) (width 0.254) (layer F.Cu) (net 14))
 (via (at 86.36 41.91) (size 0.889) (layers F.Cu B.Cu) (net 14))
 (segment (start 85.852 42.418) (end 86.36 41.91) (width 0.254) (layer B.Cu) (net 14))
 (segment (start 90.17 38.1) (end 88.265 40.005) (width 0.254) (layer F.Cu) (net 14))
 (segment (start 77.88402 41.62298) (end 78.359 41.148) (width 0.254) (layer F.Cu) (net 14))
 (segment (start 78.359 41.148) (end 80.899 41.148) (width 0.254) (layer F.Cu) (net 14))
 (segment (start 80.899 41.148) (end 82.042 40.005) (width 0.254) (layer F.Cu) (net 14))
 (segment (start 77.88402 41.62298) (end 77.88402 43.02) (width 0.254) (layer F.Cu) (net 14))
 (segment (start 82.042 40.005) (end 88.265 40.005) (width 0.254) (layer F.Cu) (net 14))
 (segment (start 78.105 42.418) (end 78.105 40.64) (width 0.254) (layer B.Cu) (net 11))
 (segment (start 81.28 39.37) (end 82.55 38.1) (width 0.254) (layer B.Cu) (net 11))
 (segment (start 79.375 39.37) (end 81.28 39.37) (width 0.254) (layer B.Cu) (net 11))
 (segment (start 78.105 40.64) (end 79.375 39.37) (width 0.254) (layer B.Cu) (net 11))
 (segment (start 75.93584 43.02) (end 75.93584 40.77716) (width 0.254) (layer F.Cu) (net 11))
 (segment (start 75.93584 40.77716) (end 76.073 40.64) (width 0.254) (layer F.Cu) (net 11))
 (segment (start 76.073 40.64) (end 76.708 40.64) (width 0.254) (layer F.Cu) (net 11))
 (segment (start 76.708 40.64) (end 77.216002 40.131998) (width 0.254) (layer F.Cu) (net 11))
 (segment (start 77.216002 40.131998) (end 80.518002 40.131998) (width 0.254) (layer F.Cu) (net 11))
 (segment (start 80.518002 40.131998) (end 82.55 38.1) (width 0.254) (layer F.Cu) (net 11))
 (segment (start 65.405 42.418) (end 61.468 42.418) (width 0.254) (layer B.Cu) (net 1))
 (segment (start 60.96 41.91) (end 57.15 38.1) (width 0.254) (layer F.Cu) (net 1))
 (via (at 60.96 41.91) (size 0.889) (layers F.Cu B.Cu) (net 1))
 (segment (start 61.468 42.418) (end 60.96 41.91) (width 0.254) (layer B.Cu) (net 1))
 (segment (start 69.43598 43.02) (end 69.43598 41.62298) (width 0.254) (layer F.Cu) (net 1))
 (segment (start 65.024 39.878) (end 58.928 39.878) (width 0.254) (layer F.Cu) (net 1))
 (segment (start 66.294 41.148) (end 65.024 39.878) (width 0.254) (layer F.Cu) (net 1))
 (segment (start 68.961 41.148) (end 66.294 41.148) (width 0.254) (layer F.Cu) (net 1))
 (segment (start 69.43598 41.62298) (end 68.961 41.148) (width 0.254) (layer F.Cu) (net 1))
 (segment (start 58.928 39.878) (end 57.15 38.1) (width 0.254) (layer F.Cu) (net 1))
 (segment (start 76.835 42.418) (end 76.835 40.64) (width 0.254) (layer B.Cu) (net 10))
 (segment (start 78.105 40.005) (end 80.01 38.1) (width 0.254) (layer B.Cu) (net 10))
 (segment (start 77.47 40.005) (end 78.105 40.005) (width 0.254) (layer B.Cu) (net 10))
 (segment (start 76.835 40.64) (end 77.47 40.005) (width 0.254) (layer B.Cu) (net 10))
 (segment (start 75.2856 43.02) (end 75.2856 40.5384) (width 0.254) (layer F.Cu) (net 10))
 (segment (start 78.613 39.497) (end 80.01 38.1) (width 0.254) (layer F.Cu) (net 10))
 (segment (start 75.2856 40.5384) (end 75.819 40.005) (width 0.254) (layer F.Cu) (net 10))
 (segment (start 75.819 40.005) (end 76.454 40.005) (width 0.254) (layer F.Cu) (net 10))
 (segment (start 76.454 40.005) (end 76.962 39.497) (width 0.254) (layer F.Cu) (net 10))
 (segment (start 76.962 39.497) (end 78.613 39.497) (width 0.254) (layer F.Cu) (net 10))
 (segment (start 65.405 49.022) (end 61.468 49.022) (width 0.254) (layer B.Cu) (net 28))
 (segment (start 60.96 49.53) (end 57.15 53.34) (width 0.254) (layer F.Cu) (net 28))
 (via (at 60.96 49.53) (size 0.889) (layers F.Cu B.Cu) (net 28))
 (segment (start 61.468 49.022) (end 60.96 49.53) (width 0.254) (layer B.Cu) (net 28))
 (segment (start 69.43598 48.42) (end 69.43598 49.81702) (width 0.254) (layer F.Cu) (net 28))
 (segment (start 64.897 51.435) (end 59.055 51.435) (width 0.254) (layer F.Cu) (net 28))
 (segment (start 66.04 50.292) (end 64.897 51.435) (width 0.254) (layer F.Cu) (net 28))
 (segment (start 68.961 50.292) (end 66.04 50.292) (width 0.254) (layer F.Cu) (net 28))
 (segment (start 69.43598 49.81702) (end 68.961 50.292) (width 0.254) (layer F.Cu) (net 28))
 (segment (start 59.055 51.435) (end 57.15 53.34) (width 0.254) (layer F.Cu) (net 28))
 (segment (start 66.675 49.022) (end 66.675 46.99) (width 0.254) (layer B.Cu) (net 27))
 (segment (start 59.69 46.99) (end 59.69 53.34) (width 0.254) (layer B.Cu) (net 27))
 (segment (start 60.325 46.355) (end 59.69 46.99) (width 0.254) (layer B.Cu) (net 27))
 (segment (start 66.04 46.355) (end 60.325 46.355) (width 0.254) (layer B.Cu) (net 27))
 (segment (start 66.675 46.99) (end 66.04 46.355) (width 0.254) (layer B.Cu) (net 27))
 (segment (start 66.421 50.8) (end 65.278 51.943) (width 0.254) (layer F.Cu) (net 27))
 (segment (start 61.087 51.943) (end 59.69 53.34) (width 0.254) (layer F.Cu) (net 27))
 (segment (start 65.278 51.943) (end 61.087 51.943) (width 0.254) (layer F.Cu) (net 27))
 (segment (start 70.08622 49.31918) (end 70.08622 50.56378) (width 0.254) (layer F.Cu) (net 27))
 (segment (start 69.85 50.8) (end 66.421 50.8) (width 0.254) (layer F.Cu) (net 27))
 (segment (start 70.08622 50.56378) (end 69.85 50.8) (width 0.254) (layer F.Cu) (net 27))
 (segment (start 67.945 49.022) (end 67.945 50.8) (width 0.254) (layer B.Cu) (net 26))
 (segment (start 67.31 51.435) (end 62.23 51.435) (width 0.254) (layer B.Cu) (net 26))
 (segment (start 67.945 50.8) (end 67.31 51.435) (width 0.254) (layer B.Cu) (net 26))
 (segment (start 62.23 53.34) (end 62.23 51.435) (width 0.254) (layer B.Cu) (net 26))
 (segment (start 62.23 51.435) (end 62.23 50.673) (width 0.254) (layer B.Cu) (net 26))
 (segment (start 62.23 50.673) (end 62.23 46.736) (width 0.254) (layer F.Cu) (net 26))
 (via (at 62.23 50.673) (size 0.889) (layers F.Cu B.Cu) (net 26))
 (segment (start 62.738 46.228) (end 62.23 46.736) (width 0.254) (layer F.Cu) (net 26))
 (segment (start 70.485 46.228) (end 62.738 46.228) (width 0.254) (layer F.Cu) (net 26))
 (segment (start 70.73392 48.42) (end 70.73392 46.34992) (width 0.254) (layer F.Cu) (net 26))
 (segment (start 70.612 46.228) (end 70.485 46.228) (width 0.254) (layer F.Cu) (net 26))
 (segment (start 70.73392 46.34992) (end 70.612 46.228) (width 0.254) (layer F.Cu) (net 26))
 (segment (start 69.215 49.022) (end 69.215 50.8) (width 0.254) (layer B.Cu) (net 25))
 (segment (start 66.04 52.07) (end 64.77 53.34) (width 0.254) (layer B.Cu) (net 25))
 (segment (start 67.945 52.07) (end 66.04 52.07) (width 0.254) (layer B.Cu) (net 25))
 (segment (start 69.215 50.8) (end 67.945 52.07) (width 0.254) (layer B.Cu) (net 25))
 (segment (start 71.38416 48.42) (end 71.38416 50.66284) (width 0.254) (layer F.Cu) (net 25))
 (segment (start 66.801998 51.308002) (end 64.77 53.34) (width 0.254) (layer F.Cu) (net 25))
 (segment (start 70.103998 51.308002) (end 66.801998 51.308002) (width 0.254) (layer F.Cu) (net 25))
 (segment (start 70.612 50.8) (end 70.103998 51.308002) (width 0.254) (layer F.Cu) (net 25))
 (segment (start 71.247 50.8) (end 70.612 50.8) (width 0.254) (layer F.Cu) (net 25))
 (segment (start 71.38416 50.66284) (end 71.247 50.8) (width 0.254) (layer F.Cu) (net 25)))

